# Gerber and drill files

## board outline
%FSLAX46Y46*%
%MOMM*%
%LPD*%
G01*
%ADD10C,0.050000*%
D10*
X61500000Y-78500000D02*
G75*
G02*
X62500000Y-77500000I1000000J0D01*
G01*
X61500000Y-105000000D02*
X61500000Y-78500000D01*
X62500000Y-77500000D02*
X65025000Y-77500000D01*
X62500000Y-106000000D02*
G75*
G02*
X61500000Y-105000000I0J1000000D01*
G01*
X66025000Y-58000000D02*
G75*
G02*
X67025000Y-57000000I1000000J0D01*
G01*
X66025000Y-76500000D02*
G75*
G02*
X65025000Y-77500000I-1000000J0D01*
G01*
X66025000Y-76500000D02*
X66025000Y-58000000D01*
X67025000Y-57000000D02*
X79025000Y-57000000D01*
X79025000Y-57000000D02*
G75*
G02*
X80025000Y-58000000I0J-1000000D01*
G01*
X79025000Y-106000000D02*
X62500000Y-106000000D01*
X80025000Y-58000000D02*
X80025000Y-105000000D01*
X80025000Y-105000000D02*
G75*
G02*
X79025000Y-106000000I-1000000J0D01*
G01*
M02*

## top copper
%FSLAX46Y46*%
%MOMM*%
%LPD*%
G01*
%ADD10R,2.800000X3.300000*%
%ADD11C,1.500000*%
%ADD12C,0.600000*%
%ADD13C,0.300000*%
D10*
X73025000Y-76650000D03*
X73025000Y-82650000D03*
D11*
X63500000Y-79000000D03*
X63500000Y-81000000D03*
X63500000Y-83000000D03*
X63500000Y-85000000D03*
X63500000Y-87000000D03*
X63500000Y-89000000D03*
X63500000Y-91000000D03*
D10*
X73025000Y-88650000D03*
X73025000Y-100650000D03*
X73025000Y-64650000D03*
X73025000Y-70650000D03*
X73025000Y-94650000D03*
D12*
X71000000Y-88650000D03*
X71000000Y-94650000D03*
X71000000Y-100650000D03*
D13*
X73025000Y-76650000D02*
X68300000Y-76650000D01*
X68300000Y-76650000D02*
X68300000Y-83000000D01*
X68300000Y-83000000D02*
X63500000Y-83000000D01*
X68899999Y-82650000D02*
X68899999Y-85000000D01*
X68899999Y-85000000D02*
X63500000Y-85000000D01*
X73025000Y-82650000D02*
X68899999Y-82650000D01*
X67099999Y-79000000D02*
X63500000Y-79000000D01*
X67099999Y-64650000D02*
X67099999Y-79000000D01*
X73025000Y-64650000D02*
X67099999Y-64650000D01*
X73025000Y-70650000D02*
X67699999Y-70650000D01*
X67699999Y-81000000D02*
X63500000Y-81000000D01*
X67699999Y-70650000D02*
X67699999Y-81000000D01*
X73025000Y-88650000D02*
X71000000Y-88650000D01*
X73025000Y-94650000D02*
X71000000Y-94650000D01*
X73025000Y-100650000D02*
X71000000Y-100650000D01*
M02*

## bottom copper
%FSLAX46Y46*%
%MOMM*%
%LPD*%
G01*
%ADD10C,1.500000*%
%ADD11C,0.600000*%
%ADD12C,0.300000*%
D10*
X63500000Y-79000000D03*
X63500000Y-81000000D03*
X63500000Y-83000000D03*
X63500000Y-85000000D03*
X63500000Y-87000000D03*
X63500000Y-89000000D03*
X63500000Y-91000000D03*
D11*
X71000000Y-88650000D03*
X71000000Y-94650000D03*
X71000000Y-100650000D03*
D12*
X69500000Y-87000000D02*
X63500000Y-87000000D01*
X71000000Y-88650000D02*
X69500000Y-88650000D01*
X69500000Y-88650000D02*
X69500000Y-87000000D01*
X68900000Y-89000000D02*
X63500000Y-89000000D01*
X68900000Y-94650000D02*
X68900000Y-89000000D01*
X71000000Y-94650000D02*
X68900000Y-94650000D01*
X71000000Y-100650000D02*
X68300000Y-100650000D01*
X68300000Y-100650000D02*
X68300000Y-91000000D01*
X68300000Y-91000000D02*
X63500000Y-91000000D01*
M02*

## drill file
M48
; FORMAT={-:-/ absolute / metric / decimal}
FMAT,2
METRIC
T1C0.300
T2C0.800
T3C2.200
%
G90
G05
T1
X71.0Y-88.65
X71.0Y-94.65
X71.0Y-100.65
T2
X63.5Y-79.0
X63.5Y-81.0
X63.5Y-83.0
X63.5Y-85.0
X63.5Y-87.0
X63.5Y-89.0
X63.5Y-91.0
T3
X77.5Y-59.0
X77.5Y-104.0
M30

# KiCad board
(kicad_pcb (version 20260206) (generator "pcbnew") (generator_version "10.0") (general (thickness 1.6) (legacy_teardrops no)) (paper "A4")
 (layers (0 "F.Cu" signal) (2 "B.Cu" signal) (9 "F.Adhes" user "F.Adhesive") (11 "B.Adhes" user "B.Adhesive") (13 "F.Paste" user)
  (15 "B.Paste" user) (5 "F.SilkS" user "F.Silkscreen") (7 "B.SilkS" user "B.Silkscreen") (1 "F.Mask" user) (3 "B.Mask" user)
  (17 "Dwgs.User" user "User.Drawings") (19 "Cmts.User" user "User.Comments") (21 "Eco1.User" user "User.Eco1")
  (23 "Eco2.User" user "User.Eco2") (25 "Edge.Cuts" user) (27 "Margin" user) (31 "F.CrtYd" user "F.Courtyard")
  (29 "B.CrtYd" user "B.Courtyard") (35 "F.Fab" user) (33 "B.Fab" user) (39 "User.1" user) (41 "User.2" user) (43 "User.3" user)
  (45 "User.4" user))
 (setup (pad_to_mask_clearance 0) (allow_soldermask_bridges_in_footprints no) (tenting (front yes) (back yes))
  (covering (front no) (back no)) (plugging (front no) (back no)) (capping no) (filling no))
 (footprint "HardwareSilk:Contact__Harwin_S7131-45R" (layer "F.Cu") (at 73.025 76.65)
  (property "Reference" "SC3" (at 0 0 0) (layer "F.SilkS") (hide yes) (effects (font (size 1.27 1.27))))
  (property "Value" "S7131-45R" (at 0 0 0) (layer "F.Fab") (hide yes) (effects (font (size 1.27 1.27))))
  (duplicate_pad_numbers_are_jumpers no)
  (pad "1" smd rect (at 0 0) (size 2.8 3.3) (layers "F.Cu" "F.Mask" "F.Paste") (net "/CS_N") (thermal_bridge_angle 45)))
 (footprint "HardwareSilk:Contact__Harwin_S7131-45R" (layer "F.Cu") (at 73.025 82.65)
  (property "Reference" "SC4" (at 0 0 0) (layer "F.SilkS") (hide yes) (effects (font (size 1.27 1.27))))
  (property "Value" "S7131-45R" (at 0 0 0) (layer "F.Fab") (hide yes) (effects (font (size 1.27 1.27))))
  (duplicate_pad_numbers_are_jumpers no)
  (pad "1" smd rect (at 0 0) (size 2.8 3.3) (layers "F.Cu" "F.Mask" "F.Paste") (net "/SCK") (thermal_bridge_angle 45)))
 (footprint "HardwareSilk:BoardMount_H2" (layer "F.Cu") (at 77.5 104)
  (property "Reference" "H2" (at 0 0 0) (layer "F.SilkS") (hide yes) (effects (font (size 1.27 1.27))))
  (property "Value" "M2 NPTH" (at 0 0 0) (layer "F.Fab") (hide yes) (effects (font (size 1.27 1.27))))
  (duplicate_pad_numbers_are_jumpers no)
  (pad "" np_thru_hole circle (at 0 0) (size 2.2 2.2) (drill 2.2) (layers "*.Cu")))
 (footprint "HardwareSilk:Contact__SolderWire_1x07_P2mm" (layer "F.Cu") (at 63.5 79)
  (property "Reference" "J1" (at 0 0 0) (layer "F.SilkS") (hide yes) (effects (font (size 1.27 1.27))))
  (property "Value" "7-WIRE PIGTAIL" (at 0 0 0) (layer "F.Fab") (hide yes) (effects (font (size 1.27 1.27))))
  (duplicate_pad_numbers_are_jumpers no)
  (pad "1" thru_hole circle (at 0 0) (size 1.5 1.5) (drill 0.8) (layers "*.Cu") (remove_unused_layers no) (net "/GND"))
  (pad "2" thru_hole circle (at 0 2) (size 1.5 1.5) (drill 0.8) (layers "*.Cu") (remove_unused_layers no) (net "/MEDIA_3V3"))
  (pad "3" thru_hole circle (at 0 4) (size 1.5 1.5) (drill 0.8) (layers "*.Cu") (remove_unused_layers no) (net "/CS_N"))
  (pad "4" thru_hole circle (at 0 6) (size 1.5 1.5) (drill 0.8) (layers "*.Cu") (remove_unused_layers no) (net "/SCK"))
  (pad "5" thru_hole circle (at 0 8) (size 1.5 1.5) (drill 0.8) (layers "*.Cu") (remove_unused_layers no) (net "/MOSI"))
  (pad "6" thru_hole circle (at 0 10) (size 1.5 1.5) (drill 0.8) (layers "*.Cu") (remove_unused_layers no) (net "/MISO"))
  (pad "7" thru_hole circle (at 0 12) (size 1.5 1.5) (drill 0.8) (layers "*.Cu") (remove_unused_layers no) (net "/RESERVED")))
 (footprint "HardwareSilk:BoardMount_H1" (layer "F.Cu") (at 77.5 59)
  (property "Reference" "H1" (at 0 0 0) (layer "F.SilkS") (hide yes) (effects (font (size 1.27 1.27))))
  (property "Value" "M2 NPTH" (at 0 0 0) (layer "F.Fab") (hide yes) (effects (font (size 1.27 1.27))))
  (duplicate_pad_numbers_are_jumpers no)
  (pad "" np_thru_hole circle (at 0 0) (size 2.2 2.2) (drill 2.2) (layers "*.Cu")))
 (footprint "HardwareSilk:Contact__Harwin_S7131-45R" (layer "F.Cu") (at 73.025 88.65)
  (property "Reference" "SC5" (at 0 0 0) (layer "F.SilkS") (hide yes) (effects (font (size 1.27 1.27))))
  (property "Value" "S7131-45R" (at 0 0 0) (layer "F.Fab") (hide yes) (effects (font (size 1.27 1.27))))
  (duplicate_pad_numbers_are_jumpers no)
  (pad "1" smd rect (at 0 0) (size 2.8 3.3) (layers "F.Cu" "F.Mask" "F.Paste") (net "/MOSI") (thermal_bridge_angle 45)))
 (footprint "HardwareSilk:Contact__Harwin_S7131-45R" (layer "F.Cu") (at 73.025 100.65)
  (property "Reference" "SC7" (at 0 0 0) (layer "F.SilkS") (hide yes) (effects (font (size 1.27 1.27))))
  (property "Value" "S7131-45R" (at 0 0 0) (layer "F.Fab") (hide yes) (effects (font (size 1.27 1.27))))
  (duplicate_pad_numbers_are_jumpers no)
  (pad "1" smd rect (at 0 0) (size 2.8 3.3) (layers "F.Cu" "F.Mask" "F.Paste") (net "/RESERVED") (thermal_bridge_angle 45)))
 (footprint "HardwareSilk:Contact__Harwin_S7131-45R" (layer "F.Cu") (at 73.025 64.65)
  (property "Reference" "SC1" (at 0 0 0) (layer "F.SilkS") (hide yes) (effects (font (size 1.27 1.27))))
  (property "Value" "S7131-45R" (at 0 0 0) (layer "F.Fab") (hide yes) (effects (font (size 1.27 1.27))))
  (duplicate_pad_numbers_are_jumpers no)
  (pad "1" smd rect (at 0 0) (size 2.8 3.3) (layers "F.Cu" "F.Mask" "F.Paste") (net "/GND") (thermal_bridge_angle 45)))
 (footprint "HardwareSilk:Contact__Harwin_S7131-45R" (layer "F.Cu") (at 73.025 70.65)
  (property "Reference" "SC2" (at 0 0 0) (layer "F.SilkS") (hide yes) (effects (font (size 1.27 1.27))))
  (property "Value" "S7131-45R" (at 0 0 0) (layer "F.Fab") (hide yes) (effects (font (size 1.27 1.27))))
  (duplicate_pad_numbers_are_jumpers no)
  (pad "1" smd rect (at 0 0) (size 2.8 3.3) (layers "F.Cu" "F.Mask" "F.Paste") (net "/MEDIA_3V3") (thermal_bridge_angle 45)))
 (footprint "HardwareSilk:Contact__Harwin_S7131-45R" (layer "F.Cu") (at 73.025 94.65)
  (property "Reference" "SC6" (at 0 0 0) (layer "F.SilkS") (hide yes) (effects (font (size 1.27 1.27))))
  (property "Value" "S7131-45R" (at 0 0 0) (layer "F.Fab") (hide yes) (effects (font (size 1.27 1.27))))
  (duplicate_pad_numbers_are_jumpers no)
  (pad "1" smd rect (at 0 0) (size 2.8 3.3) (layers "F.Cu" "F.Mask" "F.Paste") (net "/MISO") (thermal_bridge_angle 45)))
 (gr_arc (start 61.5 78.5) (mid 61.792893 77.792893) (end 62.5 77.5) (stroke (width 0.05) (type default)) (layer "Edge.Cuts"))
 (gr_line (start 61.5 105) (end 61.5 78.5) (stroke (width 0.05) (type default)) (layer "Edge.Cuts"))
 (gr_line (start 62.5 77.5) (end 65.025 77.5) (stroke (width 0.05) (type default)) (layer "Edge.Cuts"))
 (gr_arc (start 62.5 106) (mid 61.792893 105.707106) (end 61.5 105) (stroke (width 0.05) (type default)) (layer "Edge.Cuts"))
 (gr_arc (start 66.025 58) (mid 66.317893 57.292893) (end 67.025 57) (stroke (width 0.05) (type default)) (layer "Edge.Cuts"))
 (gr_arc (start 66.025 76.5) (mid 65.732107 77.207107) (end 65.025 77.5) (stroke (width 0.05) (type default)) (layer "Edge.Cuts"))
 (gr_line (start 66.025 76.5) (end 66.025 58) (stroke (width 0.05) (type default)) (layer "Edge.Cuts"))
 (gr_line (start 67.025 57) (end 79.025 57) (stroke (width 0.05) (type default)) (layer "Edge.Cuts"))
 (gr_arc (start 79.025 57) (mid 79.732106 57.292893) (end 80.025 58) (stroke (width 0.05) (type default)) (layer "Edge.Cuts"))
 (gr_line (start 79.025 106) (end 62.5 106) (stroke (width 0.05) (type default)) (layer "Edge.Cuts"))
 (gr_line (start 80.025 58) (end 80.025 105) (stroke (width 0.05) (type default)) (layer "Edge.Cuts"))
 (gr_arc (start 80.025 105) (mid 79.732106 105.707106) (end 79.025 106) (stroke (width 0.05) (type default)) (layer "Edge.Cuts"))
 (segment (start 73.025 76.65) (end 68.3 76.65) (width 0.3) (layer "F.Cu") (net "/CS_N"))
 (segment (start 68.3 76.65) (end 68.3 83) (width 0.3) (layer "F.Cu") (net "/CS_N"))
 (segment (start 68.3 83) (end 63.5 83) (width 0.3) (layer "F.Cu") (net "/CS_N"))
 (segment (start 68.899999 82.65) (end 68.899999 85) (width 0.3) (layer "F.Cu") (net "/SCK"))
 (segment (start 68.899999 85) (end 63.5 85) (width 0.3) (layer "F.Cu") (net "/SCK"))
 (segment (start 73.025 82.65) (end 68.899999 82.65) (width 0.3) (layer "F.Cu") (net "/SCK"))
 (segment (start 67.099999 79) (end 63.5 79) (width 0.3) (layer "F.Cu") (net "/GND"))
 (segment (start 67.099999 64.65) (end 67.099999 79) (width 0.3) (layer "F.Cu") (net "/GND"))
 (segment (start 73.025 64.65) (end 67.099999 64.65) (width 0.3) (layer "F.Cu") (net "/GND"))
 (segment (start 73.025 70.65) (end 67.699999 70.65) (width 0.3) (layer "F.Cu") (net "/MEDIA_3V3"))
 (segment (start 67.699999 81) (end 63.5 81) (width 0.3) (layer "F.Cu") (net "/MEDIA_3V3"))
 (segment (start 67.699999 70.65) (end 67.699999 81) (width 0.3) (layer "F.Cu") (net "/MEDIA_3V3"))
 (segment (start 73.025 88.65) (end 71 88.65) (width 0.3) (layer "F.Cu") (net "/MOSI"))
 (via (at 71 88.65) (size 0.6) (drill 0.3) (layers "F.Cu" "B.Cu") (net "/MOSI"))
 (segment (start 69.5 87) (end 63.5 87) (width 0.3) (layer "B.Cu") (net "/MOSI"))
 (segment (start 71 88.65) (end 69.5 88.65) (width 0.3) (layer "B.Cu") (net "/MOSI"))
 (segment (start 69.5 88.65) (end 69.5 87) (width 0.3) (layer "B.Cu") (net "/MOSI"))
 (segment (start 73.025 94.65) (end 71 94.65) (width 0.3) (layer "F.Cu") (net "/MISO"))
 (via (at 71 94.65) (size 0.6) (drill 0.3) (layers "F.Cu" "B.Cu") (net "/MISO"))
 (segment (start 68.9 89) (end 63.5 89) (width 0.3) (layer "B.Cu") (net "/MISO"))
 (segment (start 68.9 94.65) (end 68.9 89) (width 0.3) (layer "B.Cu") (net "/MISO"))
 (segment (start 71 94.65) (end 68.9 94.65) (width 0.3) (layer "B.Cu") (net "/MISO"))
 (segment (start 73.025 100.65) (end 71 100.65) (width 0.3) (layer "F.Cu") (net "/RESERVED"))
 (via (at 71 100.65) (size 0.6) (drill 0.3) (layers "F.Cu" "B.Cu") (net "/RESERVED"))
 (segment (start 71 100.65) (end 68.3 100.65) (width 0.3) (layer "B.Cu") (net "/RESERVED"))
 (segment (start 68.3 100.65) (end 68.3 91) (width 0.3) (layer "B.Cu") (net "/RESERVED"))
 (segment (start 68.3 91) (end 63.5 91) (width 0.3) (layer "B.Cu") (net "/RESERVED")))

